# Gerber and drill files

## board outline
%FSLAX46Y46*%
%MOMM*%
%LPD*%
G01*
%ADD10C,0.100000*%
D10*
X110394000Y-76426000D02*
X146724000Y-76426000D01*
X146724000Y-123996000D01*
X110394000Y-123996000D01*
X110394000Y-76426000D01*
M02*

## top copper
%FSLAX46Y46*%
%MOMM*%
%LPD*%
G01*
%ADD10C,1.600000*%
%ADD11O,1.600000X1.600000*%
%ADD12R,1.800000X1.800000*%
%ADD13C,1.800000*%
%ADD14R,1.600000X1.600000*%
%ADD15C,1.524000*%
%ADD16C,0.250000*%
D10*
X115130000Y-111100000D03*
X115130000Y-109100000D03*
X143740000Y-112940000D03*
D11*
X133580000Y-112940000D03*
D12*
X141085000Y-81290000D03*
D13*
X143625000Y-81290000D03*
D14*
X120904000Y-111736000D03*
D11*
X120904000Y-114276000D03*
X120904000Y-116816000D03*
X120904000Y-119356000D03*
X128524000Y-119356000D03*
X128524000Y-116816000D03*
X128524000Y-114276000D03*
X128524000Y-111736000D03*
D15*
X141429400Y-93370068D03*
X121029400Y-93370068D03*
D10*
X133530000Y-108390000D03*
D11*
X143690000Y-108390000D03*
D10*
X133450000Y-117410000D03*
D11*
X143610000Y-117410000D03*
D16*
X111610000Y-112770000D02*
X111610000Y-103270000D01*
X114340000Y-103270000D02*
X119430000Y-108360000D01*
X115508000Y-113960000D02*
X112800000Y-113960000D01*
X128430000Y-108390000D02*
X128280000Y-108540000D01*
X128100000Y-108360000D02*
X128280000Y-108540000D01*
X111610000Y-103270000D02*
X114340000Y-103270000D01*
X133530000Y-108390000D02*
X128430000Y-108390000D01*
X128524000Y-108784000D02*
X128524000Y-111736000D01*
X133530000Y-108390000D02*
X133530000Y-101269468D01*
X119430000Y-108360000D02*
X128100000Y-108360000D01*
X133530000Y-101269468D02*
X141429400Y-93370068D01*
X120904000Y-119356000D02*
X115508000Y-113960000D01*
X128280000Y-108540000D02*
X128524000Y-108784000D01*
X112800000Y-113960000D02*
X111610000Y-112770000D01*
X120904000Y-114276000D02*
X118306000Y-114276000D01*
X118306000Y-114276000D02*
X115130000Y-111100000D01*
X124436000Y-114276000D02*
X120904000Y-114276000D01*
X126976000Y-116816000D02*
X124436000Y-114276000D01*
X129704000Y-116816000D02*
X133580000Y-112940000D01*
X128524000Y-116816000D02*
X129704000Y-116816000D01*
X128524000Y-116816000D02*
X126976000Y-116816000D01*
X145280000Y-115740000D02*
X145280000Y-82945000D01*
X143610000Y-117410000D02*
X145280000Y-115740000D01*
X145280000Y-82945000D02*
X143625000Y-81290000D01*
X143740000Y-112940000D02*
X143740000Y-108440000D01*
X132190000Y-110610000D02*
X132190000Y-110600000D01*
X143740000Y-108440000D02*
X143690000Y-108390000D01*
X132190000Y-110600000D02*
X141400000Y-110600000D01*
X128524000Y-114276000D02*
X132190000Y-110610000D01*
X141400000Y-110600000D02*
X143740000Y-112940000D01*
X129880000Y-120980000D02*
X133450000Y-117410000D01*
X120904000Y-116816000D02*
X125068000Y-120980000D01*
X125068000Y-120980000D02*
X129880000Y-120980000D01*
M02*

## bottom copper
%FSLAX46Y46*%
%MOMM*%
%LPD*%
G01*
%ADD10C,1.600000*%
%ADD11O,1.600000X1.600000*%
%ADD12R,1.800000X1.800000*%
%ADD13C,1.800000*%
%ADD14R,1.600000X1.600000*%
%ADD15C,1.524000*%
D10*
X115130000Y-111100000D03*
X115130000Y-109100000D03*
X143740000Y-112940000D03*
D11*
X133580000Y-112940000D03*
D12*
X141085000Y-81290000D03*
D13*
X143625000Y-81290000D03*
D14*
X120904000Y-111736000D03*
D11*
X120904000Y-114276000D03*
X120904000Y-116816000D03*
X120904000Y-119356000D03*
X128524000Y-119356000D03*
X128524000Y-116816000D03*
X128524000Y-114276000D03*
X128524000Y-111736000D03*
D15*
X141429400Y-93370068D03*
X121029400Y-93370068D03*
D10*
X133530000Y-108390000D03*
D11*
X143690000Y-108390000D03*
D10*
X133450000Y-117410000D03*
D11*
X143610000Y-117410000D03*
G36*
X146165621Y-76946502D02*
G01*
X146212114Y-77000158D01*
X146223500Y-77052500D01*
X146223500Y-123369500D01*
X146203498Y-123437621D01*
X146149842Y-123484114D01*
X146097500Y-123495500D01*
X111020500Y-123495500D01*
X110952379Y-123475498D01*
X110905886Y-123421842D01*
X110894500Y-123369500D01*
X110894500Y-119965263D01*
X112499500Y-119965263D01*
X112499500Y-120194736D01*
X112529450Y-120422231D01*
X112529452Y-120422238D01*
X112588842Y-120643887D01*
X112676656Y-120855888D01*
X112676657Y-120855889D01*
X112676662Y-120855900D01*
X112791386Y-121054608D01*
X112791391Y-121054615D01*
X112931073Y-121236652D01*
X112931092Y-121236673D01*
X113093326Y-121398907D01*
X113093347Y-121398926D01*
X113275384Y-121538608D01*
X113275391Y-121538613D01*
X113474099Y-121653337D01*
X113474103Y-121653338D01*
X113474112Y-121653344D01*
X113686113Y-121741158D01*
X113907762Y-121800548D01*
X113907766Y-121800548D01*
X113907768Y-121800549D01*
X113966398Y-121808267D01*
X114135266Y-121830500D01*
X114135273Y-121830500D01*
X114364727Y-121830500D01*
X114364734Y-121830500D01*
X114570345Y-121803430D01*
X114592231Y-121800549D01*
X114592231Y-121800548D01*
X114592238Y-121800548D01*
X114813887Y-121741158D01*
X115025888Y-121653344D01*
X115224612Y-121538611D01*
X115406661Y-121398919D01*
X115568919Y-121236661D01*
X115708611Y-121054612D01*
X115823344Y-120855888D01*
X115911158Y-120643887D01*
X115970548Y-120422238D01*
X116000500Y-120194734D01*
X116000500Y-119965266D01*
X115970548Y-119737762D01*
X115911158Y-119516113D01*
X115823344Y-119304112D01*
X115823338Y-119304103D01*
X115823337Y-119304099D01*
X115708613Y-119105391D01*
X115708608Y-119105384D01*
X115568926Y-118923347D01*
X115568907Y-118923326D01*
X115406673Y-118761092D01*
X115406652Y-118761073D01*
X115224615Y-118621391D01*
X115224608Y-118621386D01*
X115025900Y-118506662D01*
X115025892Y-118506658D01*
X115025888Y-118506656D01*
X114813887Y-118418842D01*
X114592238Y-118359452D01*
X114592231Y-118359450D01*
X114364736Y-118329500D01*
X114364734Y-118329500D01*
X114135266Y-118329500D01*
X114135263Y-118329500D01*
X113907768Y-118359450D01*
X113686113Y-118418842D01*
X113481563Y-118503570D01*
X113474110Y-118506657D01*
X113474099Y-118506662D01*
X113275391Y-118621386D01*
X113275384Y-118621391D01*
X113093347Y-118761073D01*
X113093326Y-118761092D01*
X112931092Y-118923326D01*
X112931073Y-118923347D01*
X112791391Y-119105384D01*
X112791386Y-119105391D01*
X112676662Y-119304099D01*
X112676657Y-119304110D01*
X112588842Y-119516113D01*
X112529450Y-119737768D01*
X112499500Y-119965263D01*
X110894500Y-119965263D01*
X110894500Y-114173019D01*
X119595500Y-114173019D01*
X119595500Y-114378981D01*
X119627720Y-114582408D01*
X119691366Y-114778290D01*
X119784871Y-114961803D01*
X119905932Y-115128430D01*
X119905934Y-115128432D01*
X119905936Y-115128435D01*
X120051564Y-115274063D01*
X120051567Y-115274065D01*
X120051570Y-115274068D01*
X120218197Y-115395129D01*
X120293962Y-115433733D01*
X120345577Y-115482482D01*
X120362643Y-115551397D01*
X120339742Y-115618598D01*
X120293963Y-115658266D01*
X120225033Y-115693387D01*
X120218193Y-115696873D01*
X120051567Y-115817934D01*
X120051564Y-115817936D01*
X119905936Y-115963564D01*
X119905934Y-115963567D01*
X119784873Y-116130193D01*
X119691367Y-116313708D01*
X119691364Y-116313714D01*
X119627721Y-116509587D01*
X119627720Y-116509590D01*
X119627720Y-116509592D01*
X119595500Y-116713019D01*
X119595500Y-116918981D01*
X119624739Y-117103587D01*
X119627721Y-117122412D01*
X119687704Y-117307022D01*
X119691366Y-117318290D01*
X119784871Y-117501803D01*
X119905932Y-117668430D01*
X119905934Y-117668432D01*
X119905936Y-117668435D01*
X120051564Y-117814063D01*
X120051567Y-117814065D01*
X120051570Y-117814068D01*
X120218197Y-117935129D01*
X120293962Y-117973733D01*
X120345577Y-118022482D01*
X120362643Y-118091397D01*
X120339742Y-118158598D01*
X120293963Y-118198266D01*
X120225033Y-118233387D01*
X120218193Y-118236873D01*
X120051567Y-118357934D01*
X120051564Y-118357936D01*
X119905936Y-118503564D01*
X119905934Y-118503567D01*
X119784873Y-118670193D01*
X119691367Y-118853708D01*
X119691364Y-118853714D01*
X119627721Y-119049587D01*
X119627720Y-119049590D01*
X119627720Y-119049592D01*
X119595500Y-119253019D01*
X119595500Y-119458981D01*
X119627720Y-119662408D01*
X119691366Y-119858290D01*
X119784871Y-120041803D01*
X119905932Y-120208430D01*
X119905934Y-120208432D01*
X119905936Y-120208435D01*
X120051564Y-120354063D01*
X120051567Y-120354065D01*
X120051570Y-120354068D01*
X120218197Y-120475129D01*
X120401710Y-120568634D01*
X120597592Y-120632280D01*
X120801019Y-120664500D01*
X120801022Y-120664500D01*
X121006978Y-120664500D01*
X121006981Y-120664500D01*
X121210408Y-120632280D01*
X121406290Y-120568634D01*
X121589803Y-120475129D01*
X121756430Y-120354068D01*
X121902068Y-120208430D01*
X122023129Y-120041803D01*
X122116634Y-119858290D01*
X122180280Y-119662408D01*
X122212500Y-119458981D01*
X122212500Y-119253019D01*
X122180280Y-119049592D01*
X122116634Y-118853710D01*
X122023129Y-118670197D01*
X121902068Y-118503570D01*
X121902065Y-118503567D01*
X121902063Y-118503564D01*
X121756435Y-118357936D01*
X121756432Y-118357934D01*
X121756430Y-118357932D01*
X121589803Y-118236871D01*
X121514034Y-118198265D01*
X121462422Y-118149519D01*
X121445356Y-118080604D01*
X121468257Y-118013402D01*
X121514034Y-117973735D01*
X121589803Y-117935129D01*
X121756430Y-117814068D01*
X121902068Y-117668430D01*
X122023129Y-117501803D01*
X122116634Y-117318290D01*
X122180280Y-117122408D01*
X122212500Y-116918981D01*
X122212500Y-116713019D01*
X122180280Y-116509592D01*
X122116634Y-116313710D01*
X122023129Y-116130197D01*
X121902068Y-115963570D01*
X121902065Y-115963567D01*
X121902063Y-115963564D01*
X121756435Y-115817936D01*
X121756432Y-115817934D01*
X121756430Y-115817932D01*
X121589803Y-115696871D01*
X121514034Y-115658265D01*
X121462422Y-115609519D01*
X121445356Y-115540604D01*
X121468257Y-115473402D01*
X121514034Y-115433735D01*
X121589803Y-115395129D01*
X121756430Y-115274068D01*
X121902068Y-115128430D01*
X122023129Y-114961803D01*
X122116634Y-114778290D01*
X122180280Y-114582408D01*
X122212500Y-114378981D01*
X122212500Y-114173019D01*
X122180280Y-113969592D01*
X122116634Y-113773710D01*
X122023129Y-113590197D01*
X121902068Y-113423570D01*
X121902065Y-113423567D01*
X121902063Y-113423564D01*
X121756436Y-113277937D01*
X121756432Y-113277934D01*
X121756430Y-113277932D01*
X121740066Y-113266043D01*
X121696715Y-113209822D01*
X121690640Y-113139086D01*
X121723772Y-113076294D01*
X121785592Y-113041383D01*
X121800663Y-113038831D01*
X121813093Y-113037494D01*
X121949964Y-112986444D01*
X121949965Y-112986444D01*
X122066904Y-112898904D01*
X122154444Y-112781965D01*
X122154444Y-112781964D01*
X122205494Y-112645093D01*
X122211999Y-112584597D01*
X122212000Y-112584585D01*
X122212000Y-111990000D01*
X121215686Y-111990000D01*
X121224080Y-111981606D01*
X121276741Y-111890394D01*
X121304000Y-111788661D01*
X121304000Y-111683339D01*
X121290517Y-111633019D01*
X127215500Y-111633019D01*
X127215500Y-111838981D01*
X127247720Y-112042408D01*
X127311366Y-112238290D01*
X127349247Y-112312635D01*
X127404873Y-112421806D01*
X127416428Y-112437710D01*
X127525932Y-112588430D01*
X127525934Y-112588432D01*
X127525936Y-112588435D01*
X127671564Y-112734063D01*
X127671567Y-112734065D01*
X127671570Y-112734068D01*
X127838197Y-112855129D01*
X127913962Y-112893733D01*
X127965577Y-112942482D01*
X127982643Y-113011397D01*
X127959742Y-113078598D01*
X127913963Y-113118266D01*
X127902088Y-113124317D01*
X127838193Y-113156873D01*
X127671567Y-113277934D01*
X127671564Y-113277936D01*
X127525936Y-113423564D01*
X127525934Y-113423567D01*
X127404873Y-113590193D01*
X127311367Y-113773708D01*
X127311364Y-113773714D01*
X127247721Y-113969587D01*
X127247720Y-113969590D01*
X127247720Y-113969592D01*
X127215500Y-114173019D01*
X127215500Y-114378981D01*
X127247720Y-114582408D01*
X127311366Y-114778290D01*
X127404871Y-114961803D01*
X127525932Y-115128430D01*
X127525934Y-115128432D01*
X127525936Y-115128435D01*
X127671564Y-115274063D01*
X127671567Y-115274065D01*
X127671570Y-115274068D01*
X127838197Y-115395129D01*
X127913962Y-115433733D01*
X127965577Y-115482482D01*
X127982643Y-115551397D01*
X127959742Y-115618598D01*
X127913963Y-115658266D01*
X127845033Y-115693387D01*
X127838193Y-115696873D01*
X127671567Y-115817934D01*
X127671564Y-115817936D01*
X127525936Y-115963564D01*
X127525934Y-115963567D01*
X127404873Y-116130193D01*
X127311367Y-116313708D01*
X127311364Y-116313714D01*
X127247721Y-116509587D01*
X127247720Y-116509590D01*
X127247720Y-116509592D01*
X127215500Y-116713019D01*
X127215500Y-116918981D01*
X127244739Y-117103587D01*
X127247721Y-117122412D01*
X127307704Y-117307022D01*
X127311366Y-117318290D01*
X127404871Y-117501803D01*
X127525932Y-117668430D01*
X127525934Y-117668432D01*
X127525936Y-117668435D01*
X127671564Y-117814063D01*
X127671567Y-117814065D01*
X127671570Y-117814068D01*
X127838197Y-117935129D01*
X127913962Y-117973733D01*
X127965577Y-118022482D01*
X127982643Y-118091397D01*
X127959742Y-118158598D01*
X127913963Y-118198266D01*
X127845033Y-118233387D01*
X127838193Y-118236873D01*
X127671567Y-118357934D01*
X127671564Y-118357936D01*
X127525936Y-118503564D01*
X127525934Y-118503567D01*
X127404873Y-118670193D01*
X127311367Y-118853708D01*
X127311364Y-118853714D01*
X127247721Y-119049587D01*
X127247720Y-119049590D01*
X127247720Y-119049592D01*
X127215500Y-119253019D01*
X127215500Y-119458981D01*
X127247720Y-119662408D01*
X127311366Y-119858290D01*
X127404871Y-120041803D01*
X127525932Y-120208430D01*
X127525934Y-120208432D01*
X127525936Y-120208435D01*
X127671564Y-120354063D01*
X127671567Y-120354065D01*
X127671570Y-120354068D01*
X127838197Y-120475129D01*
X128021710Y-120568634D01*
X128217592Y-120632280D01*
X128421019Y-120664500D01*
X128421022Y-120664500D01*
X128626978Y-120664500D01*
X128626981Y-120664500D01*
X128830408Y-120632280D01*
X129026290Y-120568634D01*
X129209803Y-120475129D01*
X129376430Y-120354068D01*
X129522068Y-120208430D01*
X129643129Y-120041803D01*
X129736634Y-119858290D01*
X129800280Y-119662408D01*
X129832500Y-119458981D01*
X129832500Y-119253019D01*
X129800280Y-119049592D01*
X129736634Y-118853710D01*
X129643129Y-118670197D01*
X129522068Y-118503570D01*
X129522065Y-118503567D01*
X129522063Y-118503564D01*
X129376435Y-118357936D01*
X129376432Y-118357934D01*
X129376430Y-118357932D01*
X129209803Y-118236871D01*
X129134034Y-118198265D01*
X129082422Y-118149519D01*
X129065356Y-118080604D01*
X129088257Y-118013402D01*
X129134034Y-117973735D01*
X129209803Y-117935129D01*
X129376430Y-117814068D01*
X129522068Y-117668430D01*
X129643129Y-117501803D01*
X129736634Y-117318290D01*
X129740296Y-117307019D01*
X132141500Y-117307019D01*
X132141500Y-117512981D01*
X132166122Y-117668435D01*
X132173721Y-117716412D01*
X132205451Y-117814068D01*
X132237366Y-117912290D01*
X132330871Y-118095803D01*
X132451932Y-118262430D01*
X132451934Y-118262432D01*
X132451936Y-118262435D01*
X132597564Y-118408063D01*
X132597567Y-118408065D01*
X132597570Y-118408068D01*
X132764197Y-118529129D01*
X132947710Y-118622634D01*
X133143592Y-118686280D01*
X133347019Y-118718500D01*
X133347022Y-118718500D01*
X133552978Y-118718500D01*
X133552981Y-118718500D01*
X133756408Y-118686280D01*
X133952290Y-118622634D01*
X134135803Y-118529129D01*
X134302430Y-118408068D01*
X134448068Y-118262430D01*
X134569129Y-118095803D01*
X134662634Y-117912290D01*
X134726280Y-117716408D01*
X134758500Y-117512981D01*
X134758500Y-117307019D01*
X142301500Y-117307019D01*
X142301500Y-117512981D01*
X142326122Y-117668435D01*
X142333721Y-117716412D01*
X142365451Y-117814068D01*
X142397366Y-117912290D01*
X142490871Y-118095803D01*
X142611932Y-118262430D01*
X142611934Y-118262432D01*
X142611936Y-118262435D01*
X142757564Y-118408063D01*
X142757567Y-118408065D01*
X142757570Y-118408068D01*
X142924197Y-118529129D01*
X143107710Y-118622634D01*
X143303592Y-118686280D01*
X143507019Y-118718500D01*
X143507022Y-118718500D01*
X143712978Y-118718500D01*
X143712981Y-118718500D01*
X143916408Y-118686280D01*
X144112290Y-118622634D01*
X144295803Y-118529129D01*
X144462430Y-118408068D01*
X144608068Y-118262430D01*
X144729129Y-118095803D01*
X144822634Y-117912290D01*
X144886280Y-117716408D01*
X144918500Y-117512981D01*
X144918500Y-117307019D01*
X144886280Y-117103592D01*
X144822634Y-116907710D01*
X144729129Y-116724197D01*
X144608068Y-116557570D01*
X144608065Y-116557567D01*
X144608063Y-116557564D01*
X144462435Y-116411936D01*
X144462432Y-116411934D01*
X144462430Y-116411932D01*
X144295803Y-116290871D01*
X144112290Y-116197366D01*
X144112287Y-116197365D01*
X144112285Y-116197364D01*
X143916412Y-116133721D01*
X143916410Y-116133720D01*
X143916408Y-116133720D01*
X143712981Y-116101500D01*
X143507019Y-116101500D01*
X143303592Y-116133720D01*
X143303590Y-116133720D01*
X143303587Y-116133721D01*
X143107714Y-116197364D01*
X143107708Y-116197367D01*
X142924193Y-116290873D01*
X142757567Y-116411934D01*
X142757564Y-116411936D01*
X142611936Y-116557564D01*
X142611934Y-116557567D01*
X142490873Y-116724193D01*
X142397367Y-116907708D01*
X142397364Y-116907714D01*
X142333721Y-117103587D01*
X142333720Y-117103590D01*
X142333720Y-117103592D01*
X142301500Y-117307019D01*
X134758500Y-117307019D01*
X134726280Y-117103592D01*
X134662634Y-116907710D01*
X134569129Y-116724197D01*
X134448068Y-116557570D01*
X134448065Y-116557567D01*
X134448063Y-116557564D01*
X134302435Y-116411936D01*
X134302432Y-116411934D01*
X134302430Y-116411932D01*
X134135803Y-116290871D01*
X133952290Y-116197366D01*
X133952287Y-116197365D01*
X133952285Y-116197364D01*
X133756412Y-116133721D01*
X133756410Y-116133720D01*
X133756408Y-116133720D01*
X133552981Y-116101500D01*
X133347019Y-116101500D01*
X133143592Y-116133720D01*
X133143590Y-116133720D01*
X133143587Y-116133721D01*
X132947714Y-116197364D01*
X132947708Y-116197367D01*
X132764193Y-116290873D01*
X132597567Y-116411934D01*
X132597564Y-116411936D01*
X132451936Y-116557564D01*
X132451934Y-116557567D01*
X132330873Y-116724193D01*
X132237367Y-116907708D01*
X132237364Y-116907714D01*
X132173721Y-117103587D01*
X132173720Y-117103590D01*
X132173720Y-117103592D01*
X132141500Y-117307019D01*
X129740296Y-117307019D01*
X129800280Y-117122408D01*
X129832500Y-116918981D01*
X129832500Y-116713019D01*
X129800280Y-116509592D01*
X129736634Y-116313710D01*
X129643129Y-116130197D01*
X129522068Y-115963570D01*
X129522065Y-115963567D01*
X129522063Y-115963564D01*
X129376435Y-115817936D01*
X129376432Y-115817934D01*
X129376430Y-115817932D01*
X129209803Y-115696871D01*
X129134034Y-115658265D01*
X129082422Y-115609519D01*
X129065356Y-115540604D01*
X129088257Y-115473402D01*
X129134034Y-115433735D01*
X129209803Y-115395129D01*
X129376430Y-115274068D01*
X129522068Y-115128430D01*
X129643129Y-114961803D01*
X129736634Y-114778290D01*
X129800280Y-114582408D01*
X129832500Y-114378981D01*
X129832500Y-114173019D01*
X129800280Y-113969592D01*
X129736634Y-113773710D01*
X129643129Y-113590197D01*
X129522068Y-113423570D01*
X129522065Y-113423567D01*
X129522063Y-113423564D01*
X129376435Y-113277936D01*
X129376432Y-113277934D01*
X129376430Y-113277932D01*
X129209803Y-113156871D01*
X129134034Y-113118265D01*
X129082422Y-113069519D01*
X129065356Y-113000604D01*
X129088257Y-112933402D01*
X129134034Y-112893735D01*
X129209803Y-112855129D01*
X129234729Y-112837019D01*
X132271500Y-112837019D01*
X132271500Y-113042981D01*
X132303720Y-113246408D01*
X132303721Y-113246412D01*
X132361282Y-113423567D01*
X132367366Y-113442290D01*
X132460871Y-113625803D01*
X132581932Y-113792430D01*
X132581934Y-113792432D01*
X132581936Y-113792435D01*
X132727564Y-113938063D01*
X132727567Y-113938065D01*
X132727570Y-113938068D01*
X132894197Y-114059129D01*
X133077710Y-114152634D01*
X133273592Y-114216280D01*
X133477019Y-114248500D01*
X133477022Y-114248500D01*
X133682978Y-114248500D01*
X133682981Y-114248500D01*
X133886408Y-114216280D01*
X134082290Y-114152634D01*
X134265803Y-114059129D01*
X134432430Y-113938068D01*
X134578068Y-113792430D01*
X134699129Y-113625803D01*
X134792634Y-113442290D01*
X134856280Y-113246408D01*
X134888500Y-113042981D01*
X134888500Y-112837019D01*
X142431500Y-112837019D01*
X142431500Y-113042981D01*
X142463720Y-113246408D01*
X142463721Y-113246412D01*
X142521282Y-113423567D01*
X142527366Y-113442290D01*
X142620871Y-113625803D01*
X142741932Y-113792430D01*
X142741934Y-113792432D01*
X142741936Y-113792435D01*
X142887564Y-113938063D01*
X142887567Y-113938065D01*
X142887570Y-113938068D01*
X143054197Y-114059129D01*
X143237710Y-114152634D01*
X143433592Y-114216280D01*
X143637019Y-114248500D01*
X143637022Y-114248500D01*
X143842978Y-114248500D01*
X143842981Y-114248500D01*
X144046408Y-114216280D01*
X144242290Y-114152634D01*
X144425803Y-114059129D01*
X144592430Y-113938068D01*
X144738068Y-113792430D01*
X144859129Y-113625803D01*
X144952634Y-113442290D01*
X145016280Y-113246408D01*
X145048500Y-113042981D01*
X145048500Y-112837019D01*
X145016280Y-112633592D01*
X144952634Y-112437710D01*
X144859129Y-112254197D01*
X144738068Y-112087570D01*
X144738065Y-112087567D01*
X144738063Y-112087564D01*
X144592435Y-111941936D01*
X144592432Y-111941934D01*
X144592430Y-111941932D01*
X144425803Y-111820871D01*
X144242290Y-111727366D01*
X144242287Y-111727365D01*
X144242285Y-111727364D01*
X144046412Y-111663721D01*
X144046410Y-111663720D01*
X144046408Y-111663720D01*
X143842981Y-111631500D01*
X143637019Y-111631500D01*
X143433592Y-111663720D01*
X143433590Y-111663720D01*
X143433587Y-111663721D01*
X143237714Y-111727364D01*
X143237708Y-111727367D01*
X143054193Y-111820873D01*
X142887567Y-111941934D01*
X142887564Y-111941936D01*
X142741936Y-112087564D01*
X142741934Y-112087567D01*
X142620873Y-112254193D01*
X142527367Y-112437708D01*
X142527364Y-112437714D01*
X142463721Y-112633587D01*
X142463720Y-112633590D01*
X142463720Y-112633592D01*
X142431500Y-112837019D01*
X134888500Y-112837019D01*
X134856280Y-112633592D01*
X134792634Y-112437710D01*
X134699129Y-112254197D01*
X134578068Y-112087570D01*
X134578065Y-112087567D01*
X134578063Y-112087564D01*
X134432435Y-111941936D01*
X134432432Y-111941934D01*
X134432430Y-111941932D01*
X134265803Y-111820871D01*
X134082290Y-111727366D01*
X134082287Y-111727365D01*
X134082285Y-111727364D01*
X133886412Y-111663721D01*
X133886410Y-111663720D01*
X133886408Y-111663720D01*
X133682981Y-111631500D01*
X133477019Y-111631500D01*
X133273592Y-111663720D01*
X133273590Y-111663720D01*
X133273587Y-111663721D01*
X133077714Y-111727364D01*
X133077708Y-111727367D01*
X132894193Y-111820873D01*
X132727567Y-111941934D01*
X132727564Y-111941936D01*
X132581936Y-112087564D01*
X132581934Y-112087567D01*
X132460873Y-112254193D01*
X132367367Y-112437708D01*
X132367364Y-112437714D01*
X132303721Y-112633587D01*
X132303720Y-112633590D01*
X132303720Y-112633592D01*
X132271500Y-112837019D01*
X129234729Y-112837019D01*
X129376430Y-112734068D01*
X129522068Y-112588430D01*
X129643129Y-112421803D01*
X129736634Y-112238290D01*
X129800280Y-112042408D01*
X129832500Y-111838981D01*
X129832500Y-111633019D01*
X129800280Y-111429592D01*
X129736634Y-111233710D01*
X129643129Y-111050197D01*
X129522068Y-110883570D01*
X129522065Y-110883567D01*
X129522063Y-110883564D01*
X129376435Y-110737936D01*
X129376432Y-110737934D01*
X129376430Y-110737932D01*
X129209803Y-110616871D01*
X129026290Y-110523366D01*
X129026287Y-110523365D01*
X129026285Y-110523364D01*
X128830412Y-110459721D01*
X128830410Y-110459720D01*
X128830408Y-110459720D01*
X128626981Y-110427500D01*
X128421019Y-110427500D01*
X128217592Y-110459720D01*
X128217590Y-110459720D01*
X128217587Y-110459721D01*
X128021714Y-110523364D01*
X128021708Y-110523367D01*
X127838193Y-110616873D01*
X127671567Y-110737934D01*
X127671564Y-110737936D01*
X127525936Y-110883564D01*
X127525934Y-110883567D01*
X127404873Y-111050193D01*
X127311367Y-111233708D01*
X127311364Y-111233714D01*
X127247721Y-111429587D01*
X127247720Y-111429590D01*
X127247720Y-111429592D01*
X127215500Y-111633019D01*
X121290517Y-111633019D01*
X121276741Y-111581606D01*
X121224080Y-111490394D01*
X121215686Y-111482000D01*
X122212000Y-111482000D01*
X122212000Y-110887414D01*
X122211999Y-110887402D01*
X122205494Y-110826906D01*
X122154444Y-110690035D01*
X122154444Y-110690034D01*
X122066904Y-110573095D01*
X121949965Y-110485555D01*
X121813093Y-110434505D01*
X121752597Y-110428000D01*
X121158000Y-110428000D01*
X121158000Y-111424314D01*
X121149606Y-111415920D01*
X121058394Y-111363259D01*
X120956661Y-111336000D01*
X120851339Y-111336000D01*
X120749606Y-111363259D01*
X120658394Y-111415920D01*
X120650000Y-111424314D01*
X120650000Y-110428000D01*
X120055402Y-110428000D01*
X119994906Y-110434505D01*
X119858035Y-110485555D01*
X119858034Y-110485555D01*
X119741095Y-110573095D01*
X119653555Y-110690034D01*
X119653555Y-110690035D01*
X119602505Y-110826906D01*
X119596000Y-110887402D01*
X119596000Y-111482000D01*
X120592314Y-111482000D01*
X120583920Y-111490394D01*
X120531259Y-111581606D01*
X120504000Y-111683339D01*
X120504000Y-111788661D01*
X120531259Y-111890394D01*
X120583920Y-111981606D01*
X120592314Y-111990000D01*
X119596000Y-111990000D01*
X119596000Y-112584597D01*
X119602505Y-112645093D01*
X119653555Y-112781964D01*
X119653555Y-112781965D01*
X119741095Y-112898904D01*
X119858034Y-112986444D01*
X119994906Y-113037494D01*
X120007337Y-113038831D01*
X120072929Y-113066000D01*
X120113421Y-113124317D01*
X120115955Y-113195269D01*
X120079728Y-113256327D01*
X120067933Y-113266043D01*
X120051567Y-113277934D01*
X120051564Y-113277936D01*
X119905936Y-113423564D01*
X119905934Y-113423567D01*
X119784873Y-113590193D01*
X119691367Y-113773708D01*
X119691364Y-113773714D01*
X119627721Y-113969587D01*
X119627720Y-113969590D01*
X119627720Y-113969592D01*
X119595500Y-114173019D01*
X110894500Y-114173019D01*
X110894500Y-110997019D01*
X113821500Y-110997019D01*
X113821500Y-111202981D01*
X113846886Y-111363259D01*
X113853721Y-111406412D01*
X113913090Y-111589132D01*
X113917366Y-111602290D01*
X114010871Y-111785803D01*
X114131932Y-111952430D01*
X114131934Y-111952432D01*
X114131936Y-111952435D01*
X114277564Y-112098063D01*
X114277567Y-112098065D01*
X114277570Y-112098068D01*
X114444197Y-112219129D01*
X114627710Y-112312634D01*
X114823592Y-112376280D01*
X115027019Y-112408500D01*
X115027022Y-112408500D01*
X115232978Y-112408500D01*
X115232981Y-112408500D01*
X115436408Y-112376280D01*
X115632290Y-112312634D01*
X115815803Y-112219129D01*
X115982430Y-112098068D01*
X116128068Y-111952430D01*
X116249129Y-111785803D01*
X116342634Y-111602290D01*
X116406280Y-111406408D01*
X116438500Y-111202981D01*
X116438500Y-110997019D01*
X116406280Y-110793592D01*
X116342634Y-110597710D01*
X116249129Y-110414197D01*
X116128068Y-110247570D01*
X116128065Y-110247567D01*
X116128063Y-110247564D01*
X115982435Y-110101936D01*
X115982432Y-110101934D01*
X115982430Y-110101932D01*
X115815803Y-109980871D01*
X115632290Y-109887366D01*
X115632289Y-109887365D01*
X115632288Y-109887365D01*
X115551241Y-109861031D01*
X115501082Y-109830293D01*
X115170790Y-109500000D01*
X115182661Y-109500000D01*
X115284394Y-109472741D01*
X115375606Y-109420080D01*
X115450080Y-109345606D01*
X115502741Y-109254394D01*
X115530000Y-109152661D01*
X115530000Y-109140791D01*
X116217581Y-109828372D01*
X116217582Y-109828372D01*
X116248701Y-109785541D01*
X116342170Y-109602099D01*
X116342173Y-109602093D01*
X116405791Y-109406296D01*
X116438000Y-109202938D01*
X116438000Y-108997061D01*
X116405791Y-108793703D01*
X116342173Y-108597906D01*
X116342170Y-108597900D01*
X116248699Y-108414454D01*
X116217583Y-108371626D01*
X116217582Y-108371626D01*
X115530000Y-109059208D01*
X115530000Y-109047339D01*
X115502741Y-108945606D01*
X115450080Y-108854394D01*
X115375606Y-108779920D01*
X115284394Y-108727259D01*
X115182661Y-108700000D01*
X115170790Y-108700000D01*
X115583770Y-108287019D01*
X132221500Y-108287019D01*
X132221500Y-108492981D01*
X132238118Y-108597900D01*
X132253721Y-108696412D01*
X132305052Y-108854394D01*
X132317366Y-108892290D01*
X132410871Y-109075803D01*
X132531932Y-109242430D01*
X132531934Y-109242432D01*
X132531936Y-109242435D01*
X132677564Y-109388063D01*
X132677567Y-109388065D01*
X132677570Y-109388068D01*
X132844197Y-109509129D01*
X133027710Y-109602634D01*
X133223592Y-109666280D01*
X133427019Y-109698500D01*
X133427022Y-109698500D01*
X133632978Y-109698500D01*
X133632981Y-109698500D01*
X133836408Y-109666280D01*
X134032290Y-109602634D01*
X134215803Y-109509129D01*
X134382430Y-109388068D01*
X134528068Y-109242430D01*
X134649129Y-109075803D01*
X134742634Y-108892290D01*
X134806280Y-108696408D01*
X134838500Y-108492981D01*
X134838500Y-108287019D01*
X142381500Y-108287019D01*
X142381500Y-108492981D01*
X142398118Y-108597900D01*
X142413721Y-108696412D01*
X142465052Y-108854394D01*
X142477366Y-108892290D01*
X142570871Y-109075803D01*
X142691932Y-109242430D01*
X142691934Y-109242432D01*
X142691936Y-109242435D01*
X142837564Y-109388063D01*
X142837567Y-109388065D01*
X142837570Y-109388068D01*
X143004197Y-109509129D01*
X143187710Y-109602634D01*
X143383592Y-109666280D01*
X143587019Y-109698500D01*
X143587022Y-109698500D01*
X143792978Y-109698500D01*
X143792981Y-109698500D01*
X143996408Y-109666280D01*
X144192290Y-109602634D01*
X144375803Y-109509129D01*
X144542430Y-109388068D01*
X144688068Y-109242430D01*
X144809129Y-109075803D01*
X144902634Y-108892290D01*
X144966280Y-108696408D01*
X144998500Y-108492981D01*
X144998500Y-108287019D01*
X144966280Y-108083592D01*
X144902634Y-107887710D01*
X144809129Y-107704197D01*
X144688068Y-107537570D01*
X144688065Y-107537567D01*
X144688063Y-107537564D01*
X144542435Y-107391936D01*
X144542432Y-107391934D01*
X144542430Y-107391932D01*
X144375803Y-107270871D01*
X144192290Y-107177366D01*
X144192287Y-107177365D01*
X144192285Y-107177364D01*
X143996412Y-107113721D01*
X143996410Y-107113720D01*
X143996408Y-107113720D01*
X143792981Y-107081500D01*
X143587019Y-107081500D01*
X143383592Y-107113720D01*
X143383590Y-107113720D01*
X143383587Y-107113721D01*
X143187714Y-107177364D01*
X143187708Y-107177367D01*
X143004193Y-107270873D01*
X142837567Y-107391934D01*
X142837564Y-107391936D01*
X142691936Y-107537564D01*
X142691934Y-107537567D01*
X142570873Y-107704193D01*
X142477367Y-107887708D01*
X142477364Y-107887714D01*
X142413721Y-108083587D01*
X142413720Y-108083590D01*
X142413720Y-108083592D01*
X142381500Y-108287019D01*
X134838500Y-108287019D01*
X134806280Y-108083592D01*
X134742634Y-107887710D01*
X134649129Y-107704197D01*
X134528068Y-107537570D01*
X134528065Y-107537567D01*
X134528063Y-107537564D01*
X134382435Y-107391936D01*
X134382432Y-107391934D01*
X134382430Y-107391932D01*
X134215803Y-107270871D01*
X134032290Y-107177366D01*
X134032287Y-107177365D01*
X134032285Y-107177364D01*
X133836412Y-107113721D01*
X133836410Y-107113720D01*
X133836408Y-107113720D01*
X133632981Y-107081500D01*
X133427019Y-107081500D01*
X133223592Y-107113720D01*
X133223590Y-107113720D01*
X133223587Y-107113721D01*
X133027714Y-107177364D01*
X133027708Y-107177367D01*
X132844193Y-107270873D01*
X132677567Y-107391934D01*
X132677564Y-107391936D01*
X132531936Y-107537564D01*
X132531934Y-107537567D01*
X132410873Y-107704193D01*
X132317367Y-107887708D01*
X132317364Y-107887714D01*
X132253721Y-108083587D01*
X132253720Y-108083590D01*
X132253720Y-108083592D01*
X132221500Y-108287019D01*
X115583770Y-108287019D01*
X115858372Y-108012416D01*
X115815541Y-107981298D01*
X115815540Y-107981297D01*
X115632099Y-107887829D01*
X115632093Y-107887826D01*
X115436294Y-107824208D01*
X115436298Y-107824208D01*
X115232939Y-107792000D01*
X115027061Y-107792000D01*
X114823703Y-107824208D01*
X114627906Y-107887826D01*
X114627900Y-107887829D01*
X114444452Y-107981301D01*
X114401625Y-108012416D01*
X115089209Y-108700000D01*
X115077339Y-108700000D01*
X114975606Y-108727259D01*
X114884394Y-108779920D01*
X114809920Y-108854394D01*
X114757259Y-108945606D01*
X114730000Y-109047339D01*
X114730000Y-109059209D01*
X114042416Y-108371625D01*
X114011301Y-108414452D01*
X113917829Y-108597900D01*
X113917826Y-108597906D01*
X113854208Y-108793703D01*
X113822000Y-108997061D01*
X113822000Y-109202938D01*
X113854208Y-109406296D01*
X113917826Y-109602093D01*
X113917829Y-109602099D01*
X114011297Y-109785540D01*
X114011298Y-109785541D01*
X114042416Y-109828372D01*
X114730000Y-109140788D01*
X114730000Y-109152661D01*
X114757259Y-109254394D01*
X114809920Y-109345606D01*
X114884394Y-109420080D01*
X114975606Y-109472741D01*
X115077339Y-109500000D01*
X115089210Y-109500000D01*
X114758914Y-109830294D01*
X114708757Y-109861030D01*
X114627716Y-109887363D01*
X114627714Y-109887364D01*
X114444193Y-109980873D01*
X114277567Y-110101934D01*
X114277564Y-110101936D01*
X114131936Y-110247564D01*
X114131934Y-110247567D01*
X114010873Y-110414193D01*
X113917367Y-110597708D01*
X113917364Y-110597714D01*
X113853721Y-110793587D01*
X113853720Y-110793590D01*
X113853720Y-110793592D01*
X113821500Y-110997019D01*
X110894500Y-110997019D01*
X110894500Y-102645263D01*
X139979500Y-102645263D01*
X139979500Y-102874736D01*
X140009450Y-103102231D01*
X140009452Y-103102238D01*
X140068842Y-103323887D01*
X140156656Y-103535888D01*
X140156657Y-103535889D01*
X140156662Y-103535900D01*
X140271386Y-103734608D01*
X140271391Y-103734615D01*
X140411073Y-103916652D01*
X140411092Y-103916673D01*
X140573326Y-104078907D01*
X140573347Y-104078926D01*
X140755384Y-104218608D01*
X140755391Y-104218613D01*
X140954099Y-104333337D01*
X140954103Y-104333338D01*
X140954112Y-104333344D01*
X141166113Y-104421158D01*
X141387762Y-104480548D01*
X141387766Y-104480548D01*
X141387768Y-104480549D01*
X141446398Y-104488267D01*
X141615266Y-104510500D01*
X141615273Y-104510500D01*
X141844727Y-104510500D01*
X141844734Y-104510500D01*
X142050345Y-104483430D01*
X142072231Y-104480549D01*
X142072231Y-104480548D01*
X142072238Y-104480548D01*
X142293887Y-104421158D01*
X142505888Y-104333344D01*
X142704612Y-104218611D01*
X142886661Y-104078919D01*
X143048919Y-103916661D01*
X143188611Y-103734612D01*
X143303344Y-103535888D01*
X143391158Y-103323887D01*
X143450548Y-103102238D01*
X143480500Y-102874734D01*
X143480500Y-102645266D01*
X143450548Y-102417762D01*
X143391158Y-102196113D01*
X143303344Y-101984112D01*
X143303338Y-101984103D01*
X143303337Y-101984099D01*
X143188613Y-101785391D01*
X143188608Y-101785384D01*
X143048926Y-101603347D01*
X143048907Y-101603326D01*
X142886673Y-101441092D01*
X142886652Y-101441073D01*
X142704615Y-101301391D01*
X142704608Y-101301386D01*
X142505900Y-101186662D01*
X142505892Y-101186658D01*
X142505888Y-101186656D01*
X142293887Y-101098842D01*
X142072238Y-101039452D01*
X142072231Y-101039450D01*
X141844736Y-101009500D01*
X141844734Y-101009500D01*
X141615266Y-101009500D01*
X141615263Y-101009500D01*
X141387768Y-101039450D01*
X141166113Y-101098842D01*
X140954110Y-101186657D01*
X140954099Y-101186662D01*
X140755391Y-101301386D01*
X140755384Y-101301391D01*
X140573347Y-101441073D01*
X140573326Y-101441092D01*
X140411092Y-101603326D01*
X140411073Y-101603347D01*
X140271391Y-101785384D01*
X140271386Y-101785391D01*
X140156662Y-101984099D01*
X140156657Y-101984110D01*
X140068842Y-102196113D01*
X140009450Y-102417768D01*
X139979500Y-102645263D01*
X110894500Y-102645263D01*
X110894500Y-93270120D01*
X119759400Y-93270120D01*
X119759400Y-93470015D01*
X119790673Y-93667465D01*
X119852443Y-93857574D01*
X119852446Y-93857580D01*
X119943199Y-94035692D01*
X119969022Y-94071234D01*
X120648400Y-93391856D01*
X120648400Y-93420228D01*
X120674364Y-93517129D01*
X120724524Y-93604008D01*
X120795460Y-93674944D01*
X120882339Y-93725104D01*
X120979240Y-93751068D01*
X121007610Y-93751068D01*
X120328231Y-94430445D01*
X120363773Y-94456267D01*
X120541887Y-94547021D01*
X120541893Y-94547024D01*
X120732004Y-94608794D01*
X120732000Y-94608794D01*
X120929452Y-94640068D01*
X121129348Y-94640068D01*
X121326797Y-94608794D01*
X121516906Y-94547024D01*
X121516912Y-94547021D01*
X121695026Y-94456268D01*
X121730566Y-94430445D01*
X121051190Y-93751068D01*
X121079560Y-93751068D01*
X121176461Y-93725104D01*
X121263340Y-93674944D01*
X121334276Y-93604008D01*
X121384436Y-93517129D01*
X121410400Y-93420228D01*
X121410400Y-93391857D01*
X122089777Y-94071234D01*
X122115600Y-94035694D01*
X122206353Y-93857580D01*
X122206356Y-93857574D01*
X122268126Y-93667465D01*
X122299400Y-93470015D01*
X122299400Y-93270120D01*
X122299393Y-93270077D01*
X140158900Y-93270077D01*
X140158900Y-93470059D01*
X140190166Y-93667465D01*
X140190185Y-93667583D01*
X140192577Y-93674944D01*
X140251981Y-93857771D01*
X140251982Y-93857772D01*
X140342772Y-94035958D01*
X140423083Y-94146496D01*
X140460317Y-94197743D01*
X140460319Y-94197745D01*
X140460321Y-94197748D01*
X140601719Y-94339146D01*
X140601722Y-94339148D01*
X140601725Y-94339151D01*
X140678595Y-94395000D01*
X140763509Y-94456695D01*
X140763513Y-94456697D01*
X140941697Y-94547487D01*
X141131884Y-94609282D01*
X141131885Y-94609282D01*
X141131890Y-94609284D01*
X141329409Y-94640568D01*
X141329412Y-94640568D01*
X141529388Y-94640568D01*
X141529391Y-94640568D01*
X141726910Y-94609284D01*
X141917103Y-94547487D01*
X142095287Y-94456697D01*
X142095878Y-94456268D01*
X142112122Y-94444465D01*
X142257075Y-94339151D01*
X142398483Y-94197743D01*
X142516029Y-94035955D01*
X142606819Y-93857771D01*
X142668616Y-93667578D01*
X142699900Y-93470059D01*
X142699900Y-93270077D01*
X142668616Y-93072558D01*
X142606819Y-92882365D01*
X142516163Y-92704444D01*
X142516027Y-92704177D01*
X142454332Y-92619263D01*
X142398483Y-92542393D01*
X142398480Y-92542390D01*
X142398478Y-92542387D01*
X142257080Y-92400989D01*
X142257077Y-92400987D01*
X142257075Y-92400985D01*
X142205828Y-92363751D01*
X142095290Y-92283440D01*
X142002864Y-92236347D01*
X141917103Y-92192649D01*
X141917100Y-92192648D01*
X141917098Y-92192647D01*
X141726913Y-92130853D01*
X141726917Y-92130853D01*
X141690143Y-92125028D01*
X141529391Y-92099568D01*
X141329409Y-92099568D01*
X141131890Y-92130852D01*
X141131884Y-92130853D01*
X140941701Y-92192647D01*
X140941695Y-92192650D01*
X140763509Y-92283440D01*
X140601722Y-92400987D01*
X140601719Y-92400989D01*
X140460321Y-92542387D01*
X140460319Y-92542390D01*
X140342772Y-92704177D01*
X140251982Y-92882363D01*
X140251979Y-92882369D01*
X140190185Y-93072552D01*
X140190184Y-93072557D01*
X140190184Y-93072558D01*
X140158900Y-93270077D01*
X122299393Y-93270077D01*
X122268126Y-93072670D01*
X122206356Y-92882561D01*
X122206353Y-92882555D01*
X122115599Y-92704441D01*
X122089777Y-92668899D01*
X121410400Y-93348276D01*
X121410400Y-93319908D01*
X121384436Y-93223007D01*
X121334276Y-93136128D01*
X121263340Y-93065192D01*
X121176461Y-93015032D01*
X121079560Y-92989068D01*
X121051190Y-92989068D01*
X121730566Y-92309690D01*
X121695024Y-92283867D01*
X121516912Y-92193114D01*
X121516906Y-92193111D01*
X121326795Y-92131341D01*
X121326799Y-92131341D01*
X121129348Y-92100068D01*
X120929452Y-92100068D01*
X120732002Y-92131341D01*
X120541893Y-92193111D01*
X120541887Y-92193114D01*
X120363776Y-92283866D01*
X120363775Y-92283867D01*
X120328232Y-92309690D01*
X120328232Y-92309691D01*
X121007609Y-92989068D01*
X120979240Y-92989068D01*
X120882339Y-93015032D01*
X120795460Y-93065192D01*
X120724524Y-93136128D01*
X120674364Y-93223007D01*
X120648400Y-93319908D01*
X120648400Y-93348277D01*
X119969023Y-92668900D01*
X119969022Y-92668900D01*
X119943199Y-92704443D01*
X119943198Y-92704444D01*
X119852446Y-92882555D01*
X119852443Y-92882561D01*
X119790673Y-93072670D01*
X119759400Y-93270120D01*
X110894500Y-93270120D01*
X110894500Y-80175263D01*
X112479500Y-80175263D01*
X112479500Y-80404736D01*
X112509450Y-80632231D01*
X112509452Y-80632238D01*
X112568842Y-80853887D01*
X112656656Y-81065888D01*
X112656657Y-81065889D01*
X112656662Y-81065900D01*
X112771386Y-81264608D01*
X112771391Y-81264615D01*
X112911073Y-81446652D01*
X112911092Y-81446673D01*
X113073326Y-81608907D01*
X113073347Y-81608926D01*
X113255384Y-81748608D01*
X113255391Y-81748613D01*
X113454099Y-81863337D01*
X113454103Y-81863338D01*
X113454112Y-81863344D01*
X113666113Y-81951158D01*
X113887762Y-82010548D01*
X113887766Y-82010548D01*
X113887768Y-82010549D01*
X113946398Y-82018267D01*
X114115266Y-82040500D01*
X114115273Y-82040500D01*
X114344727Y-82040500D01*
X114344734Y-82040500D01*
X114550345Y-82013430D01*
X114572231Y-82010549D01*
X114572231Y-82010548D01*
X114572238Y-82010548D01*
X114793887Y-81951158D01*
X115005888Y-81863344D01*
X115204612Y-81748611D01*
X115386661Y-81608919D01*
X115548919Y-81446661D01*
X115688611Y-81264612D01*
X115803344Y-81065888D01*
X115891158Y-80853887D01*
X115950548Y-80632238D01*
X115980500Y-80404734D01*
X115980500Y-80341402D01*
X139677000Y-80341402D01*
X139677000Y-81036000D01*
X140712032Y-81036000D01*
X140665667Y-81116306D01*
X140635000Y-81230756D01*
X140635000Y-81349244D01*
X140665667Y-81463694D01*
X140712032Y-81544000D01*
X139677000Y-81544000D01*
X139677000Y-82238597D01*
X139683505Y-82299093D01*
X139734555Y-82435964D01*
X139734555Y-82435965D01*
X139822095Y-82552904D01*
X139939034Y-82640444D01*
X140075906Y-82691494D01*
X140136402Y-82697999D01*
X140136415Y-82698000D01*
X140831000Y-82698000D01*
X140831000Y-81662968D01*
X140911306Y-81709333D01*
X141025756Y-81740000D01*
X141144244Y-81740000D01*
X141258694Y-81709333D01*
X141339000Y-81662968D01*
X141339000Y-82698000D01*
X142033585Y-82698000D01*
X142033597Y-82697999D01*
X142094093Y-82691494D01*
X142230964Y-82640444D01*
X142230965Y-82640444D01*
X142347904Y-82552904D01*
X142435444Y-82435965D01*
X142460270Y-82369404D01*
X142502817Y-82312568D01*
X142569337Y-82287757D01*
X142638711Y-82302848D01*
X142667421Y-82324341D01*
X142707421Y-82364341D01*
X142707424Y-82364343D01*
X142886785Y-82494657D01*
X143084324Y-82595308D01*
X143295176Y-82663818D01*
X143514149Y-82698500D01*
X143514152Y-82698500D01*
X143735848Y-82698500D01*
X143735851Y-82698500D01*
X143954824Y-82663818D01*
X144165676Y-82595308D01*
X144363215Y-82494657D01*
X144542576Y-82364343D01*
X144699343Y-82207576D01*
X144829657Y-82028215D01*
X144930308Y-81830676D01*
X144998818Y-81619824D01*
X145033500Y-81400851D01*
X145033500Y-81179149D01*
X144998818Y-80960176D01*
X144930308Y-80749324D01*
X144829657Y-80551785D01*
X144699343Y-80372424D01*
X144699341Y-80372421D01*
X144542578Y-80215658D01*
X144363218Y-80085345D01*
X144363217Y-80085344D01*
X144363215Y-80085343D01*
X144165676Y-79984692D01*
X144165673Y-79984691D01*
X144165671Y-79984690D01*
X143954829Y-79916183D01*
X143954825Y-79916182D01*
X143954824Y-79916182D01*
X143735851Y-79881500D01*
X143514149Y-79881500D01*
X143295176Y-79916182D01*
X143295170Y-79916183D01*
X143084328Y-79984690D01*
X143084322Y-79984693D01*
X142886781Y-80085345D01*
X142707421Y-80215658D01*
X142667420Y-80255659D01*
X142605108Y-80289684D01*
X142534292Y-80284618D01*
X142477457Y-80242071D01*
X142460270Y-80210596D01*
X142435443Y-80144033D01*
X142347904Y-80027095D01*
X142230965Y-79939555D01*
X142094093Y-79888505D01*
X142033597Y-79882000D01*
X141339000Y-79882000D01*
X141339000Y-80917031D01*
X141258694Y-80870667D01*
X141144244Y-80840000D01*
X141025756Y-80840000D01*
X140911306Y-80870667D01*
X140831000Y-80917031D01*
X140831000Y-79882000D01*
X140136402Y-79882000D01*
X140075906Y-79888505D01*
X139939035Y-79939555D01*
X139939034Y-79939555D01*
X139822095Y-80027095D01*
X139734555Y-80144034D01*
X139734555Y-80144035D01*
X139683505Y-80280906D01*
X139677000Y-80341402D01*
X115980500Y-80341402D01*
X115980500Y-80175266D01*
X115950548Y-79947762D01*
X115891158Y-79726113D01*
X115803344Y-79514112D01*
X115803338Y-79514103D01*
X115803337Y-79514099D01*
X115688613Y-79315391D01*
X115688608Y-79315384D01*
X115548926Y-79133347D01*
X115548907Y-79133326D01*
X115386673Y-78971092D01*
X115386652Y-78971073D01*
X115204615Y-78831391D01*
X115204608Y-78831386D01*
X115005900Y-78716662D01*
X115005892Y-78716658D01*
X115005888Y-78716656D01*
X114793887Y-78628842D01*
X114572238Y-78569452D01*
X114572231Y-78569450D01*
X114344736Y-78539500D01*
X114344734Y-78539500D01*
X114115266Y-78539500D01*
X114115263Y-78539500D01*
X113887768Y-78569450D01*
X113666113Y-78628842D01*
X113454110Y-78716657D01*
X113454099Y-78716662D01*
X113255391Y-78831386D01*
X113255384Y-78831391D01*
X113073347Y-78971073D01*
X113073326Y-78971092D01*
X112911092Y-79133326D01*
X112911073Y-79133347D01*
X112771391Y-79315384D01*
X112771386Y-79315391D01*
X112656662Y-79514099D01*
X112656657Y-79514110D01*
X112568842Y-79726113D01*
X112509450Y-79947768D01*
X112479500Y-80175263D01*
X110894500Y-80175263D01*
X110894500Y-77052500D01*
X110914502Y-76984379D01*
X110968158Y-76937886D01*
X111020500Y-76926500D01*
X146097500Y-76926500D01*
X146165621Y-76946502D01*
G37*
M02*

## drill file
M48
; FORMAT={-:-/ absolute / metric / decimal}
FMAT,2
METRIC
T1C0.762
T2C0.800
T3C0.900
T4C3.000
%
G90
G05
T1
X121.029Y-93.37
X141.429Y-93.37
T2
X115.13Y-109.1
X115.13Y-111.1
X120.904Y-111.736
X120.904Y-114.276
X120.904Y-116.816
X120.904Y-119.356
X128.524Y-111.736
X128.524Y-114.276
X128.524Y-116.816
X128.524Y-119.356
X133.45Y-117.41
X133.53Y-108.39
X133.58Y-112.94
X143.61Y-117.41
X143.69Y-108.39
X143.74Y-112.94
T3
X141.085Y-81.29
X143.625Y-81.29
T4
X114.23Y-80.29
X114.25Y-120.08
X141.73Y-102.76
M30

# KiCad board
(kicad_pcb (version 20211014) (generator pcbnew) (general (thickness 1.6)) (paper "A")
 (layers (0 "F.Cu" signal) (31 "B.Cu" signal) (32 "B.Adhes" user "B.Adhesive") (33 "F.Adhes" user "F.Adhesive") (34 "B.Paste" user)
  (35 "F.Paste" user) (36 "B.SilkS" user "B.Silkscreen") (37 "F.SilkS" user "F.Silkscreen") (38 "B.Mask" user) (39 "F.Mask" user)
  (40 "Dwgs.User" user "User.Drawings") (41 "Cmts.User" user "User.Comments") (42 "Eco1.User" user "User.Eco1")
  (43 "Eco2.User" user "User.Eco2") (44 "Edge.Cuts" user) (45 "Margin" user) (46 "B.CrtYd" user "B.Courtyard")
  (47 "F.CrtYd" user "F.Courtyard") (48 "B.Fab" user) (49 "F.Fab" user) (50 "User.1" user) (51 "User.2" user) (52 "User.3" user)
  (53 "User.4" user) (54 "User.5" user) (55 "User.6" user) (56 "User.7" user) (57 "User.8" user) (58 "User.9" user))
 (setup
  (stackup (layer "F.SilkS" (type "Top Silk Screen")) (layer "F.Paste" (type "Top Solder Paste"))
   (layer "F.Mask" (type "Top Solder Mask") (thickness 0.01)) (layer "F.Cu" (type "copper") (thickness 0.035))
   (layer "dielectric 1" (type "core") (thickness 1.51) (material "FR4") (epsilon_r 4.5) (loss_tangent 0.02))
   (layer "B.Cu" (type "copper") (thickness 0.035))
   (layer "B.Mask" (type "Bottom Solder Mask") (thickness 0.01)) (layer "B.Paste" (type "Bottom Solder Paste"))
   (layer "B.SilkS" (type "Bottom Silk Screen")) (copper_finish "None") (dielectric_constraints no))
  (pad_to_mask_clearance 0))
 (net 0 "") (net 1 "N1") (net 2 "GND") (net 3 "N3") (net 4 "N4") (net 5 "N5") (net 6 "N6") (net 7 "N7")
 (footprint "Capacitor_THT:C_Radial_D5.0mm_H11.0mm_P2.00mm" (layer "F.Cu") (at 115.13 111.1 90)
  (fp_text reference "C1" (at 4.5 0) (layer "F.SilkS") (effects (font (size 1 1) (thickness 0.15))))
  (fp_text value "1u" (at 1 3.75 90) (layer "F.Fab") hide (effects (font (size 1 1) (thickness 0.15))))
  (pad "1" thru_hole circle (at 0 0 90) (size 1.6 1.6) (drill 0.8) (layers *.Cu *.Mask) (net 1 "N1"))
  (pad "2" thru_hole circle (at 2 0 90) (size 1.6 1.6) (drill 0.8) (layers *.Cu *.Mask) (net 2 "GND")))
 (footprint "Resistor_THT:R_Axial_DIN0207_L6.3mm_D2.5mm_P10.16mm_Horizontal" (layer "F.Cu") (at 143.74 112.94 180)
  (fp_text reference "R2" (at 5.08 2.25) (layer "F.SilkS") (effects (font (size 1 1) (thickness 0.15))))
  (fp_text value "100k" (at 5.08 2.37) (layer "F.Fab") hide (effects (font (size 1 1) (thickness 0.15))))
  (pad "1" thru_hole circle (at 0 0 180) (size 1.6 1.6) (drill 0.8) (layers *.Cu *.Mask) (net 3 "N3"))
  (pad "2" thru_hole oval (at 10.16 0 180) (size 1.6 1.6) (drill 0.8) (layers *.Cu *.Mask) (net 1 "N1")))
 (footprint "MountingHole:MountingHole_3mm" (layer "F.Cu") (at 141.73 102.76)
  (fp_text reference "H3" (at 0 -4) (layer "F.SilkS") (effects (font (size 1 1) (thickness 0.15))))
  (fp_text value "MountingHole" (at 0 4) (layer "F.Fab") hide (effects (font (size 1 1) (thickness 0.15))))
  (pad "" np_thru_hole circle (at 0 0) (size 3 3) (drill 3) (layers *.Cu *.Mask)))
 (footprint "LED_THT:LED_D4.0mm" (layer "F.Cu") (at 141.085 81.29)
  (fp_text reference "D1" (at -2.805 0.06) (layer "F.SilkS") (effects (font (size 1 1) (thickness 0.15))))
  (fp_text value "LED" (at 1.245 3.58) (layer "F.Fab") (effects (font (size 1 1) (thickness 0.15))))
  (pad "1" thru_hole rect (at 0 0) (size 1.8 1.8) (drill 0.9) (layers *.Cu *.Mask) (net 2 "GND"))
  (pad "2" thru_hole circle (at 2.54 0) (size 1.8 1.8) (drill 0.9) (layers *.Cu *.Mask) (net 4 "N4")))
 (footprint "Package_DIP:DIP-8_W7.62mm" (layer "F.Cu") (at 120.904 111.736)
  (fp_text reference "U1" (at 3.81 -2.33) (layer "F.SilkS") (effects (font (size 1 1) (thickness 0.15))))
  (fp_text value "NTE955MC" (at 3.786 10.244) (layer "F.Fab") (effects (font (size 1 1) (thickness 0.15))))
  (pad "1" thru_hole rect (at 0 0) (size 1.6 1.6) (drill 0.8) (layers *.Cu *.Mask) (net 2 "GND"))
  (pad "2" thru_hole oval (at 0 2.54) (size 1.6 1.6) (drill 0.8) (layers *.Cu *.Mask) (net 1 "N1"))
  (pad "3" thru_hole oval (at 0 5.08) (size 1.6 1.6) (drill 0.8) (layers *.Cu *.Mask) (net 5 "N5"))
  (pad "4" thru_hole oval (at 0 7.62) (size 1.6 1.6) (drill 0.8) (layers *.Cu *.Mask) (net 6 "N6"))
  (pad "5" thru_hole oval (at 7.62 7.62) (size 1.6 1.6) (drill 0.8) (layers *.Cu *.Mask) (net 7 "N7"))
  (pad "6" thru_hole oval (at 7.62 5.08) (size 1.6 1.6) (drill 0.8) (layers *.Cu *.Mask) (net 1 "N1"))
  (pad "7" thru_hole oval (at 7.62 2.54) (size 1.6 1.6) (drill 0.8) (layers *.Cu *.Mask) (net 3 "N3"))
  (pad "8" thru_hole oval (at 7.62 0) (size 1.6 1.6) (drill 0.8) (layers *.Cu *.Mask) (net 6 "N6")))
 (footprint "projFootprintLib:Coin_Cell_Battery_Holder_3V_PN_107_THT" (layer "F.Cu") (at 126.4294 93.370068 180)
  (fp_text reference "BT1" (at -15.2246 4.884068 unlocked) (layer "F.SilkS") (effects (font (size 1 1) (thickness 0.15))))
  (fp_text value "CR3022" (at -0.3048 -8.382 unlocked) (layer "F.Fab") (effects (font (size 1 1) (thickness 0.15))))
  (pad "1" thru_hole circle (at -15 0 180) (size 1.524 1.524) (drill 0.762) (layers *.Cu *.Mask) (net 6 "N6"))
  (pad "2" thru_hole circle (at 5.4 0 180) (size 1.524 1.524) (drill 0.762) (layers *.Cu *.Mask) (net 2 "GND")))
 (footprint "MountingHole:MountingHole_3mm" (layer "F.Cu") (at 114.25 120.08)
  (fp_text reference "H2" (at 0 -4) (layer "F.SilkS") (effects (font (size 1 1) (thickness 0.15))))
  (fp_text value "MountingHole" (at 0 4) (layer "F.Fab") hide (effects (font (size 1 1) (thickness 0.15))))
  (pad "" np_thru_hole circle (at 0 0) (size 3 3) (drill 3) (layers *.Cu *.Mask)))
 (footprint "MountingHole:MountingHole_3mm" (layer "F.Cu") (at 114.23 80.29)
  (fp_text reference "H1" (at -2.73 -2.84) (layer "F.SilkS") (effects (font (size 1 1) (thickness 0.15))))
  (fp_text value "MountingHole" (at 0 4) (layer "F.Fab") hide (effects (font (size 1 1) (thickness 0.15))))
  (pad "" np_thru_hole circle (at 0 0) (size 3 3) (drill 3) (layers *.Cu *.Mask)))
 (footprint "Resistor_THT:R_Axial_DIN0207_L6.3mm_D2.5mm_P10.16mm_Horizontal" (layer "F.Cu") (at 133.53 108.39)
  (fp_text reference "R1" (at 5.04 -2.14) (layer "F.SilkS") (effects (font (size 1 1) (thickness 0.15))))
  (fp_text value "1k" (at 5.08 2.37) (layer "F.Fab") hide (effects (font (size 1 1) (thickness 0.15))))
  (pad "1" thru_hole circle (at 0 0) (size 1.6 1.6) (drill 0.8) (layers *.Cu *.Mask) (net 6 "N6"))
  (pad "2" thru_hole oval (at 10.16 0) (size 1.6 1.6) (drill 0.8) (layers *.Cu *.Mask) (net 3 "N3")))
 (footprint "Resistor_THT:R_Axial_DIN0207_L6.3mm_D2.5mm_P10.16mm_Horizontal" (layer "F.Cu") (at 133.45 117.41)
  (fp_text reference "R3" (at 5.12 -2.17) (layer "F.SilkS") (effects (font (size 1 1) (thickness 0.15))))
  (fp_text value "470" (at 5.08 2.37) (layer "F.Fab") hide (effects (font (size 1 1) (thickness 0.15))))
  (pad "1" thru_hole circle (at 0 0) (size 1.6 1.6) (drill 0.8) (layers *.Cu *.Mask) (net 5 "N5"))
  (pad "2" thru_hole oval (at 10.16 0) (size 1.6 1.6) (drill 0.8) (layers *.Cu *.Mask) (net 4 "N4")))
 (gr_rect (start 110.394 76.426) (end 146.724 123.996) (layer "Edge.Cuts") (width 0.1) (fill none))
 (segment (start 111.61 112.77) (end 111.61 103.27) (width 0.25) (layer "F.Cu") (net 6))
 (segment (start 114.34 103.27) (end 119.43 108.36) (width 0.25) (layer "F.Cu") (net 6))
 (segment (start 115.508 113.96) (end 112.8 113.96) (width 0.25) (layer "F.Cu") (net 6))
 (segment (start 128.43 108.39) (end 128.28 108.54) (width 0.25) (layer "F.Cu") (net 6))
 (segment (start 128.1 108.36) (end 128.28 108.54) (width 0.25) (layer "F.Cu") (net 6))
 (segment (start 111.61 103.27) (end 114.34 103.27) (width 0.25) (layer "F.Cu") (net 6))
 (segment (start 133.53 108.39) (end 128.43 108.39) (width 0.25) (layer "F.Cu") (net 6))
 (segment (start 128.524 108.784) (end 128.524 111.736) (width 0.25) (layer "F.Cu") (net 6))
 (segment (start 133.53 108.39) (end 133.53 101.269468) (width 0.25) (layer "F.Cu") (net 6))
 (segment (start 119.43 108.36) (end 128.1 108.36) (width 0.25) (layer "F.Cu") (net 6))
 (segment (start 133.53 101.269468) (end 141.4294 93.370068) (width 0.25) (layer "F.Cu") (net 6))
 (segment (start 120.904 119.356) (end 115.508 113.96) (width 0.25) (layer "F.Cu") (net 6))
 (segment (start 128.28 108.54) (end 128.524 108.784) (width 0.25) (layer "F.Cu") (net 6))
 (segment (start 112.8 113.96) (end 111.61 112.77) (width 0.25) (layer "F.Cu") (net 6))
 (segment (start 120.904 114.276) (end 118.306 114.276) (width 0.25) (layer "F.Cu") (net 1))
 (segment (start 118.306 114.276) (end 115.13 111.1) (width 0.25) (layer "F.Cu") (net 1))
 (segment (start 124.436 114.276) (end 120.904 114.276) (width 0.25) (layer "F.Cu") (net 1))
 (segment (start 126.976 116.816) (end 124.436 114.276) (width 0.25) (layer "F.Cu") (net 1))
 (segment (start 129.704 116.816) (end 133.58 112.94) (width 0.25) (layer "F.Cu") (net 1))
 (segment (start 128.524 116.816) (end 129.704 116.816) (width 0.25) (layer "F.Cu") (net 1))
 (segment (start 128.524 116.816) (end 126.976 116.816) (width 0.25) (layer "F.Cu") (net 1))
 (segment (start 145.28 115.74) (end 145.28 82.945) (width 0.25) (layer "F.Cu") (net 4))
 (segment (start 143.61 117.41) (end 145.28 115.74) (width 0.25) (layer "F.Cu") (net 4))
 (segment (start 145.28 82.945) (end 143.625 81.29) (width 0.25) (layer "F.Cu") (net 4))
 (segment (start 143.74 112.94) (end 143.74 108.44) (width 0.25) (layer "F.Cu") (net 3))
 (segment (start 132.19 110.61) (end 132.19 110.6) (width 0.25) (layer "F.Cu") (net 3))
 (segment (start 143.74 108.44) (end 143.69 108.39) (width 0.25) (layer "F.Cu") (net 3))
 (segment (start 132.19 110.6) (end 141.4 110.6) (width 0.25) (layer "F.Cu") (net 3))
 (segment (start 128.524 114.276) (end 132.19 110.61) (width 0.25) (layer "F.Cu") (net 3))
 (segment (start 141.4 110.6) (end 143.74 112.94) (width 0.25) (layer "F.Cu") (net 3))
 (segment (start 129.88 120.98) (end 133.45 117.41) (width 0.25) (layer "F.Cu") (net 5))
 (segment (start 120.904 116.816) (end 125.068 120.98) (width 0.25) (layer "F.Cu") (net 5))
 (segment (start 125.068 120.98) (end 129.88 120.98) (width 0.25) (layer "F.Cu") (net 5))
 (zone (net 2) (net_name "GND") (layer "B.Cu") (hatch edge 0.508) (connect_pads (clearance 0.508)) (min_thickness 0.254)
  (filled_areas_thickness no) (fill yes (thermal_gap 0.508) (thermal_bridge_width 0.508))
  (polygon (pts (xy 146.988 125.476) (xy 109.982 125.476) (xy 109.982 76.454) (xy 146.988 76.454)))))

